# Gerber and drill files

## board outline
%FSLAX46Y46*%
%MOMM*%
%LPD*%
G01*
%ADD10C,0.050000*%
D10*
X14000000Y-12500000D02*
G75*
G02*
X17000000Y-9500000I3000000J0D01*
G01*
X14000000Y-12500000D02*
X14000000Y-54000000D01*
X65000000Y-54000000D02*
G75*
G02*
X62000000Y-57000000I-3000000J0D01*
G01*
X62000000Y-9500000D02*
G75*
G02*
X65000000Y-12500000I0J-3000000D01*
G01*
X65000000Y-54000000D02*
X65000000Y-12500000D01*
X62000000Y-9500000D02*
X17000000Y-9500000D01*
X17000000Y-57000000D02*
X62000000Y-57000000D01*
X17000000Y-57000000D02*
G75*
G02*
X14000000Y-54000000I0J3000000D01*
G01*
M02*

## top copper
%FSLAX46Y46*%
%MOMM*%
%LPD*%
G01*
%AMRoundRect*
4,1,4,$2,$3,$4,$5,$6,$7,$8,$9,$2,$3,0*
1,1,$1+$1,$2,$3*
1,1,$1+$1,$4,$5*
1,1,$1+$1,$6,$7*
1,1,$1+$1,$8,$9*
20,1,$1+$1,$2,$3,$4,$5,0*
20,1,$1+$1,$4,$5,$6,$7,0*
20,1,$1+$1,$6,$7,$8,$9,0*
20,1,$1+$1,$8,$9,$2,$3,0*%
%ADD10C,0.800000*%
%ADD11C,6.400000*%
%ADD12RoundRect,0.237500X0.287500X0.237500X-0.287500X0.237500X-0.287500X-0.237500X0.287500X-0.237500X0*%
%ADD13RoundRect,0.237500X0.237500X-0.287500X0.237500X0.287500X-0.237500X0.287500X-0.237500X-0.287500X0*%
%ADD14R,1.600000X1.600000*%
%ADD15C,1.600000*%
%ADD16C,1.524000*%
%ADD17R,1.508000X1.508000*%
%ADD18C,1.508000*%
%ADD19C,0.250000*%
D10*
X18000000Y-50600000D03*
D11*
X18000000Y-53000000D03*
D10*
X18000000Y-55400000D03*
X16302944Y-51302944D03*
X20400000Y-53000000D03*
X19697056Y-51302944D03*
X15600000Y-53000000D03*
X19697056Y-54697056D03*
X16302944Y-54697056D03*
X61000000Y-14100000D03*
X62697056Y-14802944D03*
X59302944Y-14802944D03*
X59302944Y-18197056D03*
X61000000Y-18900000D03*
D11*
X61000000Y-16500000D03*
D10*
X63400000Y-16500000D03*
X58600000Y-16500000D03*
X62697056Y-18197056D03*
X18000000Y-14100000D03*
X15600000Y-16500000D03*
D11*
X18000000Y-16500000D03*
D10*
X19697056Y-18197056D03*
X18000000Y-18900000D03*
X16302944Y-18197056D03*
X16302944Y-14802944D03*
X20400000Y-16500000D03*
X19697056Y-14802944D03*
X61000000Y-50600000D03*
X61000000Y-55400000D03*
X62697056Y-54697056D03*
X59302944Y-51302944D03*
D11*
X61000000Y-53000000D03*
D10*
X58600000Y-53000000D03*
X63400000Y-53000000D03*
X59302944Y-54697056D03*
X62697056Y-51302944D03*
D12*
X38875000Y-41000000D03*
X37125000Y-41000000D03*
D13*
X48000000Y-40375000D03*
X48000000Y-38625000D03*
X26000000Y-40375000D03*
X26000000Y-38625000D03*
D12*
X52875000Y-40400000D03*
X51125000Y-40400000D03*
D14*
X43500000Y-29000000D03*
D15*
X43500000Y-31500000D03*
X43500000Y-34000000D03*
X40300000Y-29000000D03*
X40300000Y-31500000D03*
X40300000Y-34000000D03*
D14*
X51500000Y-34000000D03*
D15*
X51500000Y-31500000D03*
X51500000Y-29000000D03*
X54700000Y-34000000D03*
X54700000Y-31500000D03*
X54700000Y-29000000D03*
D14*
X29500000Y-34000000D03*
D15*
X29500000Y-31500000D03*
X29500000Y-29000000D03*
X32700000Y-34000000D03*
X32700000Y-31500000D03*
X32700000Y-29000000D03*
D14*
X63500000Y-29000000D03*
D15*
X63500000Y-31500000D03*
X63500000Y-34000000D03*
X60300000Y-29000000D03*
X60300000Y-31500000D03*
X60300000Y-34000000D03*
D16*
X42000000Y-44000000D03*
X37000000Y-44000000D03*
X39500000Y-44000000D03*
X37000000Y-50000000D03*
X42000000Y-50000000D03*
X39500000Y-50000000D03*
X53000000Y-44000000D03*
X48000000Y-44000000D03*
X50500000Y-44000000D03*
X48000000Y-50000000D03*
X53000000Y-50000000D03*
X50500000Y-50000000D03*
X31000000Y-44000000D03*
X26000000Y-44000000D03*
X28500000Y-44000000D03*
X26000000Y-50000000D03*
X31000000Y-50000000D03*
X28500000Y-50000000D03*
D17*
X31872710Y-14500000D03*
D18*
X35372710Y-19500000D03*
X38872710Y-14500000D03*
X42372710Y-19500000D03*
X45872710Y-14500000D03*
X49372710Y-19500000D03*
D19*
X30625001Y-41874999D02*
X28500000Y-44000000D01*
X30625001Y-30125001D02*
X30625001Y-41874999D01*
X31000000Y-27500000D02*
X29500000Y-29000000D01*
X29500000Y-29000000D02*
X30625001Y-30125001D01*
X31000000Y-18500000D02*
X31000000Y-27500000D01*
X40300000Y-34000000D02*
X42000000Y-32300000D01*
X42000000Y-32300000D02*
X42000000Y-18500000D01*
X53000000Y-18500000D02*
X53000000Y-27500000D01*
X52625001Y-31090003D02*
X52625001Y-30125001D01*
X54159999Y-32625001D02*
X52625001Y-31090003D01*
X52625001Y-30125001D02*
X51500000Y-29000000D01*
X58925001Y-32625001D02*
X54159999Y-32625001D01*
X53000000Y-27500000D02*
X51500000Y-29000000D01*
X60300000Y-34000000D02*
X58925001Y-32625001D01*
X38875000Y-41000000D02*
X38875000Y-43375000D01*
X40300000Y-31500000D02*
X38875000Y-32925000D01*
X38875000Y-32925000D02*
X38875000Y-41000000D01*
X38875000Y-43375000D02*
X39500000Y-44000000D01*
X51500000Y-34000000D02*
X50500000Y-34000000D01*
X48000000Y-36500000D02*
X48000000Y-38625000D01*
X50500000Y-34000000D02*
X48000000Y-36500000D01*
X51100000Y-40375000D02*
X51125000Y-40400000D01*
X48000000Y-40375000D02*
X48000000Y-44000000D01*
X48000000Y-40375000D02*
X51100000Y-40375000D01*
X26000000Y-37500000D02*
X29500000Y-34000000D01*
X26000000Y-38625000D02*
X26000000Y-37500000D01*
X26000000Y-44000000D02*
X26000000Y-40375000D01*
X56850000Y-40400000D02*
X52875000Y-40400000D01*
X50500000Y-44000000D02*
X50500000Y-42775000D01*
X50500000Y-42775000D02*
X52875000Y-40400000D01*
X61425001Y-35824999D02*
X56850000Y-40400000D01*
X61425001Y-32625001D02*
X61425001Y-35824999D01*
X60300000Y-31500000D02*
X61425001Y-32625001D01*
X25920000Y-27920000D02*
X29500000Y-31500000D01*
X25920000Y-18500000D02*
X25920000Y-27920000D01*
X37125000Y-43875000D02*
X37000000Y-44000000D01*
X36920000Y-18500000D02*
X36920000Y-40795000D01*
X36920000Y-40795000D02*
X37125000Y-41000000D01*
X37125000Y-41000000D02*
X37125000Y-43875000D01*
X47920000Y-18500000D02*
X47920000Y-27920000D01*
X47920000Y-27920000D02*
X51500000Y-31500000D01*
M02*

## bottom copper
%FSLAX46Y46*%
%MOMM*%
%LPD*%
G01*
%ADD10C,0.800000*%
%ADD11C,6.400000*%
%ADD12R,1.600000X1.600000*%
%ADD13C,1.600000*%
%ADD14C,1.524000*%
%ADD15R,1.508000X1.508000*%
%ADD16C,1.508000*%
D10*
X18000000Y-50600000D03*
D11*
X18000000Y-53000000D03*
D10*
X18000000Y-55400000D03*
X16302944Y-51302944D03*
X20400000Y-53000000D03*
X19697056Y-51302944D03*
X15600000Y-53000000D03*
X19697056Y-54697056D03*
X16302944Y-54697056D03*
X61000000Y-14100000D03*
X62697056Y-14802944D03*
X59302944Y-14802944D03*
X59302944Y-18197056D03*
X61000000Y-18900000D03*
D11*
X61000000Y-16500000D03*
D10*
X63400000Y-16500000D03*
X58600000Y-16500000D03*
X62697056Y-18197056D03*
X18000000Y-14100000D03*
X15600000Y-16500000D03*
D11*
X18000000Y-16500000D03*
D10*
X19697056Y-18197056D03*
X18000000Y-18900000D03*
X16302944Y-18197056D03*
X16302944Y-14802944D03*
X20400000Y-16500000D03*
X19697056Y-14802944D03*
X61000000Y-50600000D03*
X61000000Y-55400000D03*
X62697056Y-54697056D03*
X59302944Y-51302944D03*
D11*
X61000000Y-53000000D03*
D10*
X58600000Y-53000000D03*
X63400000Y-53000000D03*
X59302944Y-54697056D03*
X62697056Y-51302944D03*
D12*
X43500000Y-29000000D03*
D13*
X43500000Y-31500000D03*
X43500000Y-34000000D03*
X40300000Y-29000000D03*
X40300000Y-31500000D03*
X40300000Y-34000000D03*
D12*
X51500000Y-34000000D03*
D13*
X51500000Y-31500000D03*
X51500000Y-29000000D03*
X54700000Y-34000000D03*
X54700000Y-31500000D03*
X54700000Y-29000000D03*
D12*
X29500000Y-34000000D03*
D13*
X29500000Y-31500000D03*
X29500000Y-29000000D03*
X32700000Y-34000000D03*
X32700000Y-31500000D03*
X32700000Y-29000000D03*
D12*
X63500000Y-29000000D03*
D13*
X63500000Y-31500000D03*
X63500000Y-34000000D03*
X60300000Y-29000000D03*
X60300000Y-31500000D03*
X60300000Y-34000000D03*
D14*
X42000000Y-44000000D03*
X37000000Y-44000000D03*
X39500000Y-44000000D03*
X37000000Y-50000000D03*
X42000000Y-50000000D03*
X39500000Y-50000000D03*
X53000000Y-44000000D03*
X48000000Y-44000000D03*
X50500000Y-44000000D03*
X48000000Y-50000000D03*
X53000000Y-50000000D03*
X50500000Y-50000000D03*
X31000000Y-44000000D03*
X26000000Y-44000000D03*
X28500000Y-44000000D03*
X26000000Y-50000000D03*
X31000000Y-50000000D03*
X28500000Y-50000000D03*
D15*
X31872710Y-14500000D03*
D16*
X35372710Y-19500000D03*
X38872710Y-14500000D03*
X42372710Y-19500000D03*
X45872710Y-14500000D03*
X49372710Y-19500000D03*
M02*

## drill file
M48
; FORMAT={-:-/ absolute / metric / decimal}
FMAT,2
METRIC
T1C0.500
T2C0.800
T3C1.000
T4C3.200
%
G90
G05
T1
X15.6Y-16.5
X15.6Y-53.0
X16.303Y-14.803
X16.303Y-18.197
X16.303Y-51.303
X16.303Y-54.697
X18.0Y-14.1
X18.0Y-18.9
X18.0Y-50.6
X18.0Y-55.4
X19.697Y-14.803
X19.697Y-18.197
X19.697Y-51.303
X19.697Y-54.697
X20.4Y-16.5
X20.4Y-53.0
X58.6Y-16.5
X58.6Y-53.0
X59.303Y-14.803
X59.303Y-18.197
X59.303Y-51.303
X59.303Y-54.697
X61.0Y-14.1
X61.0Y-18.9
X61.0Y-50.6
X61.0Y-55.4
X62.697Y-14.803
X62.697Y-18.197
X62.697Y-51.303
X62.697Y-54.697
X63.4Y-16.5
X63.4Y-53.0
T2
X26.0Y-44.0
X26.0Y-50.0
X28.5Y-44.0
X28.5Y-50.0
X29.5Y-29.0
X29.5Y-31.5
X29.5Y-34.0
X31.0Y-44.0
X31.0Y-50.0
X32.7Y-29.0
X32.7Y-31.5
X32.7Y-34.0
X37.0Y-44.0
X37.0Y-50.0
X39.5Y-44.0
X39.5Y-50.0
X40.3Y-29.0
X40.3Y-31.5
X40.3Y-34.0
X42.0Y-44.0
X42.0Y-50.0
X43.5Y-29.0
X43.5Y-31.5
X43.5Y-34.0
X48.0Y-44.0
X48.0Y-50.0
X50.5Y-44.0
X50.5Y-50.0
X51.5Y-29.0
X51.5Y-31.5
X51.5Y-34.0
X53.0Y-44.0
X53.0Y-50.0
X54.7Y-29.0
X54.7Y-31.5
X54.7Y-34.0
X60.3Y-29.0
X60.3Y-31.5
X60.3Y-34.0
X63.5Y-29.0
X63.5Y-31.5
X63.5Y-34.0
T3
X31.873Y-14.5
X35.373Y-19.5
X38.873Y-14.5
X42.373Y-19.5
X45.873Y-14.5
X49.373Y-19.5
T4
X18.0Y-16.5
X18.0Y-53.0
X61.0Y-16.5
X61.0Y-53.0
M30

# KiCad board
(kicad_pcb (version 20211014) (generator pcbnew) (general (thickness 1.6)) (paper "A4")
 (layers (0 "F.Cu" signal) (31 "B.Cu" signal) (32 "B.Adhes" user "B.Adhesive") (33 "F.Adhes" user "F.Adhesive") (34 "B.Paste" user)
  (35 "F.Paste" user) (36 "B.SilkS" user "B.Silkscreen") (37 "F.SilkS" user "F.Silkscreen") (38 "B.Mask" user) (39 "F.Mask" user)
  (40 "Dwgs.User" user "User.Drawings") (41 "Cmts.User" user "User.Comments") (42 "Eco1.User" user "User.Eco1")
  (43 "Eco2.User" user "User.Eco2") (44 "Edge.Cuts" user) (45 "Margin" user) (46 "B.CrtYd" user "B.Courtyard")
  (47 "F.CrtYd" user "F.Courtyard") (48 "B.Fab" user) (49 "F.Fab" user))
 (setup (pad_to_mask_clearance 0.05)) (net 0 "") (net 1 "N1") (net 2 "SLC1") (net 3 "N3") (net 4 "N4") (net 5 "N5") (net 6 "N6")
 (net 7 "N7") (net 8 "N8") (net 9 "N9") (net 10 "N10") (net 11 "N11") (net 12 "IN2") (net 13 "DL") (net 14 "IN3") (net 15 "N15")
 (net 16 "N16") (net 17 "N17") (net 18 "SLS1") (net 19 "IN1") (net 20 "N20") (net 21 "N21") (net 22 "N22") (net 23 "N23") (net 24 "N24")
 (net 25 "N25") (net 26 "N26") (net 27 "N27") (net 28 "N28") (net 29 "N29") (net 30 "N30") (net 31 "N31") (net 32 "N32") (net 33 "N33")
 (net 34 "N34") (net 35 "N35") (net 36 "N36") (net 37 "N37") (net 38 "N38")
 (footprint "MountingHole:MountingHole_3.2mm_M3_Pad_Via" (layer "F.Cu") (at 18 53)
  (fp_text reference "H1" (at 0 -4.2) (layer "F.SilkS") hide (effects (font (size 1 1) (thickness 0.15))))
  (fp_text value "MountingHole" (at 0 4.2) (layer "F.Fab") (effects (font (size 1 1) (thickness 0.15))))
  (pad "1" thru_hole circle locked (at 0 -2.4) (size 0.8 0.8) (drill 0.5) (layers *.Cu *.Mask))
  (pad "1" thru_hole circle locked (at 0 0) (size 6.4 6.4) (drill 3.2) (layers *.Cu *.Mask))
  (pad "1" thru_hole circle locked (at 0 2.4) (size 0.8 0.8) (drill 0.5) (layers *.Cu *.Mask))
  (pad "1" thru_hole circle locked (at -1.697056 -1.697056) (size 0.8 0.8) (drill 0.5) (layers *.Cu *.Mask))
  (pad "1" thru_hole circle locked (at 2.4 0) (size 0.8 0.8) (drill 0.5) (layers *.Cu *.Mask))
  (pad "1" thru_hole circle locked (at 1.697056 -1.697056) (size 0.8 0.8) (drill 0.5) (layers *.Cu *.Mask))
  (pad "1" thru_hole circle locked (at -2.4 0) (size 0.8 0.8) (drill 0.5) (layers *.Cu *.Mask))
  (pad "1" thru_hole circle locked (at 1.697056 1.697056) (size 0.8 0.8) (drill 0.5) (layers *.Cu *.Mask))
  (pad "1" thru_hole circle locked (at -1.697056 1.697056) (size 0.8 0.8) (drill 0.5) (layers *.Cu *.Mask)))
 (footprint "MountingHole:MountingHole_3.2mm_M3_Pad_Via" (layer "F.Cu") (at 61 16.5)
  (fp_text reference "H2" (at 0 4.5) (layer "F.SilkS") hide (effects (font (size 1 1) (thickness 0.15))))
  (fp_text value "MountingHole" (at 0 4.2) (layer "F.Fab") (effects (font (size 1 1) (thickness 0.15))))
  (pad "1" thru_hole circle locked (at 0 -2.4) (size 0.8 0.8) (drill 0.5) (layers *.Cu *.Mask))
  (pad "1" thru_hole circle locked (at 1.697056 -1.697056) (size 0.8 0.8) (drill 0.5) (layers *.Cu *.Mask))
  (pad "1" thru_hole circle locked (at -1.697056 -1.697056) (size 0.8 0.8) (drill 0.5) (layers *.Cu *.Mask))
  (pad "1" thru_hole circle locked (at -1.697056 1.697056) (size 0.8 0.8) (drill 0.5) (layers *.Cu *.Mask))
  (pad "1" thru_hole circle locked (at 0 2.4) (size 0.8 0.8) (drill 0.5) (layers *.Cu *.Mask))
  (pad "1" thru_hole circle locked (at 0 0) (size 6.4 6.4) (drill 3.2) (layers *.Cu *.Mask))
  (pad "1" thru_hole circle locked (at 2.4 0) (size 0.8 0.8) (drill 0.5) (layers *.Cu *.Mask))
  (pad "1" thru_hole circle locked (at -2.4 0) (size 0.8 0.8) (drill 0.5) (layers *.Cu *.Mask))
  (pad "1" thru_hole circle locked (at 1.697056 1.697056) (size 0.8 0.8) (drill 0.5) (layers *.Cu *.Mask)))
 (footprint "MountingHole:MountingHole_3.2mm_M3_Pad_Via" (layer "F.Cu") (at 18 16.5)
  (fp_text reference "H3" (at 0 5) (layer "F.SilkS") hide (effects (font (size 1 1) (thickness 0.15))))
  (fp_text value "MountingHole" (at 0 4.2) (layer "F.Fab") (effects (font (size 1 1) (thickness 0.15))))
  (pad "1" thru_hole circle locked (at 0 -2.4) (size 0.8 0.8) (drill 0.5) (layers *.Cu *.Mask))
  (pad "1" thru_hole circle locked (at -2.4 0) (size 0.8 0.8) (drill 0.5) (layers *.Cu *.Mask))
  (pad "1" thru_hole circle locked (at 0 0) (size 6.4 6.4) (drill 3.2) (layers *.Cu *.Mask))
  (pad "1" thru_hole circle locked (at 1.697056 1.697056) (size 0.8 0.8) (drill 0.5) (layers *.Cu *.Mask))
  (pad "1" thru_hole circle locked (at 0 2.4) (size 0.8 0.8) (drill 0.5) (layers *.Cu *.Mask))
  (pad "1" thru_hole circle locked (at -1.697056 1.697056) (size 0.8 0.8) (drill 0.5) (layers *.Cu *.Mask))
  (pad "1" thru_hole circle locked (at -1.697056 -1.697056) (size 0.8 0.8) (drill 0.5) (layers *.Cu *.Mask))
  (pad "1" thru_hole circle locked (at 2.4 0) (size 0.8 0.8) (drill 0.5) (layers *.Cu *.Mask))
  (pad "1" thru_hole circle locked (at 1.697056 -1.697056) (size 0.8 0.8) (drill 0.5) (layers *.Cu *.Mask)))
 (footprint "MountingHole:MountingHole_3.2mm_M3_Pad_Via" (layer "F.Cu") (at 61 53)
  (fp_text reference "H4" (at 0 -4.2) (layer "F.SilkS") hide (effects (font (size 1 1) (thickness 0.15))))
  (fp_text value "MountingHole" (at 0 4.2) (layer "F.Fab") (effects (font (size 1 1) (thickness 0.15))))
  (pad "1" thru_hole circle locked (at 0 -2.4) (size 0.8 0.8) (drill 0.5) (layers *.Cu *.Mask))
  (pad "1" thru_hole circle locked (at 0 2.4) (size 0.8 0.8) (drill 0.5) (layers *.Cu *.Mask))
  (pad "1" thru_hole circle locked (at 1.697056 1.697056) (size 0.8 0.8) (drill 0.5) (layers *.Cu *.Mask))
  (pad "1" thru_hole circle locked (at -1.697056 -1.697056) (size 0.8 0.8) (drill 0.5) (layers *.Cu *.Mask))
  (pad "1" thru_hole circle locked (at 0 0) (size 6.4 6.4) (drill 3.2) (layers *.Cu *.Mask))
  (pad "1" thru_hole circle locked (at -2.4 0) (size 0.8 0.8) (drill 0.5) (layers *.Cu *.Mask))
  (pad "1" thru_hole circle locked (at 2.4 0) (size 0.8 0.8) (drill 0.5) (layers *.Cu *.Mask))
  (pad "1" thru_hole circle locked (at -1.697056 1.697056) (size 0.8 0.8) (drill 0.5) (layers *.Cu *.Mask))
  (pad "1" thru_hole circle locked (at 1.697056 -1.697056) (size 0.8 0.8) (drill 0.5) (layers *.Cu *.Mask)))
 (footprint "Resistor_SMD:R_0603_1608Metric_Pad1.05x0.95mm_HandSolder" (layer "F.Cu") (at 38 41 180)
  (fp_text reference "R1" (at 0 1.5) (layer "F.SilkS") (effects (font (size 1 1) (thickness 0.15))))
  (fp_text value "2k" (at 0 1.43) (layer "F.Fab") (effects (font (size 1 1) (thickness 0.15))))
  (pad "1" smd roundrect locked (at -0.875 0 180) (size 1.05 0.95) (layers "F.Cu" "F.Paste" "F.Mask") (roundrect_rratio 0.25) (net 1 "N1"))
  (pad "2" smd roundrect locked (at 0.875 0 180) (size 1.05 0.95) (layers "F.Cu" "F.Paste" "F.Mask") (roundrect_rratio 0.25) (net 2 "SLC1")))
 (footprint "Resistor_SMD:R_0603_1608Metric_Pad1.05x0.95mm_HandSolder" (layer "F.Cu") (at 48 39.5 90)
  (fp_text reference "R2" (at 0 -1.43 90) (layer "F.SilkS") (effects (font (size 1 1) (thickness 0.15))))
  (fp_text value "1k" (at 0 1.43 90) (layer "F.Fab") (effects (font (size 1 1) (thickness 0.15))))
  (pad "1" smd roundrect locked (at -0.875 0 90) (size 1.05 0.95) (layers "F.Cu" "F.Paste" "F.Mask") (roundrect_rratio 0.25) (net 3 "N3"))
  (pad "2" smd roundrect locked (at 0.875 0 90) (size 1.05 0.95) (layers "F.Cu" "F.Paste" "F.Mask") (roundrect_rratio 0.25) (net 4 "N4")))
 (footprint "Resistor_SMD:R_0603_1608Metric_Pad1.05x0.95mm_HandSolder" (layer "F.Cu") (at 26 39.5 90)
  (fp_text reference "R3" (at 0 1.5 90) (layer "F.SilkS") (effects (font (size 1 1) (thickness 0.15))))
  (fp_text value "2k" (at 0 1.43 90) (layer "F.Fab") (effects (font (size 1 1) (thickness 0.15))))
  (pad "1" smd roundrect locked (at -0.875 0 90) (size 1.05 0.95) (layers "F.Cu" "F.Paste" "F.Mask") (roundrect_rratio 0.25) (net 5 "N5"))
  (pad "2" smd roundrect locked (at 0.875 0 90) (size 1.05 0.95) (layers "F.Cu" "F.Paste" "F.Mask") (roundrect_rratio 0.25) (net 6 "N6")))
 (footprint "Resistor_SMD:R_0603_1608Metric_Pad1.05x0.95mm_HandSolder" (layer "F.Cu") (at 52 40.4 180)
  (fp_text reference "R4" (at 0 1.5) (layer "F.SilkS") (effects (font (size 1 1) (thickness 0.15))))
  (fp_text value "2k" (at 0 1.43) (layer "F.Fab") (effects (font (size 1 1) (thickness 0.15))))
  (pad "1" smd roundrect locked (at -0.875 0 180) (size 1.05 0.95) (layers "F.Cu" "F.Paste" "F.Mask") (roundrect_rratio 0.25) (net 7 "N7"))
  (pad "2" smd roundrect locked (at 0.875 0 180) (size 1.05 0.95) (layers "F.Cu" "F.Paste" "F.Mask") (roundrect_rratio 0.25) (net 3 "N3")))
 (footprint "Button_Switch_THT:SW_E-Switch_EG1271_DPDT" (layer "F.Cu") (at 43.5 29 -90)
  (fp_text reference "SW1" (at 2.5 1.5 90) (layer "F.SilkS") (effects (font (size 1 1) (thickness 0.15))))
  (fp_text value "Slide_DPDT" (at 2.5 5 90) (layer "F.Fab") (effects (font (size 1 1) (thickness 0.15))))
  (pad "1" thru_hole rect locked (at 0 0 270) (size 1.6 1.6) (drill 0.8) (layers *.Cu *.Mask) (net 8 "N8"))
  (pad "2" thru_hole circle locked (at 2.5 0 270) (size 1.6 1.6) (drill 0.8) (layers *.Cu *.Mask) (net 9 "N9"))
  (pad "3" thru_hole circle locked (at 5 0 270) (size 1.6 1.6) (drill 0.8) (layers *.Cu *.Mask) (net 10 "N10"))
  (pad "4" thru_hole circle locked (at 0 3.2 270) (size 1.6 1.6) (drill 0.8) (layers *.Cu *.Mask) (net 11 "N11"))
  (pad "5" thru_hole circle locked (at 2.5 3.2 270) (size 1.6 1.6) (drill 0.8) (layers *.Cu *.Mask) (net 1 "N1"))
  (pad "6" thru_hole circle locked (at 5 3.2 270) (size 1.6 1.6) (drill 0.8) (layers *.Cu *.Mask) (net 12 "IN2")))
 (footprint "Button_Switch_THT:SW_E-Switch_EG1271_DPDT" (layer "F.Cu") (at 51.5 34 90)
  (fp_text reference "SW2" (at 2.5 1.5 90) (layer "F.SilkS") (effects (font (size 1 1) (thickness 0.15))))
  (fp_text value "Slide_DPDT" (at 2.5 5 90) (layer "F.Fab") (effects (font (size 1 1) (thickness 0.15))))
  (pad "1" thru_hole rect locked (at 0 0 90) (size 1.6 1.6) (drill 0.8) (layers *.Cu *.Mask) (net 4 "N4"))
  (pad "2" thru_hole circle locked (at 2.5 0 90) (size 1.6 1.6) (drill 0.8) (layers *.Cu *.Mask) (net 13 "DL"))
  (pad "3" thru_hole circle locked (at 5 0 90) (size 1.6 1.6) (drill 0.8) (layers *.Cu *.Mask) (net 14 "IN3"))
  (pad "4" thru_hole circle locked (at 0 3.2 90) (size 1.6 1.6) (drill 0.8) (layers *.Cu *.Mask) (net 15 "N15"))
  (pad "5" thru_hole circle locked (at 2.5 3.2 90) (size 1.6 1.6) (drill 0.8) (layers *.Cu *.Mask) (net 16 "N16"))
  (pad "6" thru_hole circle locked (at 5 3.2 90) (size 1.6 1.6) (drill 0.8) (layers *.Cu *.Mask) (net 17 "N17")))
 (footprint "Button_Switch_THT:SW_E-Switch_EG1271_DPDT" (layer "F.Cu") (at 29.5 34 90)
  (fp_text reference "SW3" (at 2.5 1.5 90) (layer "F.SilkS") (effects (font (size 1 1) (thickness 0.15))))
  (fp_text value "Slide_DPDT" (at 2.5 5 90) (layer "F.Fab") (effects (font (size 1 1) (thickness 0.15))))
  (pad "1" thru_hole rect locked (at 0 0 90) (size 1.6 1.6) (drill 0.8) (layers *.Cu *.Mask) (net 6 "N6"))
  (pad "2" thru_hole circle locked (at 2.5 0 90) (size 1.6 1.6) (drill 0.8) (layers *.Cu *.Mask) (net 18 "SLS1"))
  (pad "3" thru_hole circle locked (at 5 0 90) (size 1.6 1.6) (drill 0.8) (layers *.Cu *.Mask) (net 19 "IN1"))
  (pad "4" thru_hole circle locked (at 0 3.2 90) (size 1.6 1.6) (drill 0.8) (layers *.Cu *.Mask) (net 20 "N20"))
  (pad "5" thru_hole circle locked (at 2.5 3.2 90) (size 1.6 1.6) (drill 0.8) (layers *.Cu *.Mask) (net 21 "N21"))
  (pad "6" thru_hole circle locked (at 5 3.2 90) (size 1.6 1.6) (drill 0.8) (layers *.Cu *.Mask) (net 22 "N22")))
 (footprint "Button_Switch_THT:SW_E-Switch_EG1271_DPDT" (layer "F.Cu") (at 63.5 29 -90)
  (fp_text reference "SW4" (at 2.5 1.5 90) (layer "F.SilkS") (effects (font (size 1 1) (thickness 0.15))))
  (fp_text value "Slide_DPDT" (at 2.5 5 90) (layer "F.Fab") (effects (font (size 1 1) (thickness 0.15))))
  (pad "1" thru_hole rect locked (at 0 0 270) (size 1.6 1.6) (drill 0.8) (layers *.Cu *.Mask) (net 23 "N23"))
  (pad "2" thru_hole circle locked (at 2.5 0 270) (size 1.6 1.6) (drill 0.8) (layers *.Cu *.Mask) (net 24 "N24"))
  (pad "3" thru_hole circle locked (at 5 0 270) (size 1.6 1.6) (drill 0.8) (layers *.Cu *.Mask) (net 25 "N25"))
  (pad "4" thru_hole circle locked (at 0 3.2 270) (size 1.6 1.6) (drill 0.8) (layers *.Cu *.Mask) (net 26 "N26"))
  (pad "5" thru_hole circle locked (at 2.5 3.2 270) (size 1.6 1.6) (drill 0.8) (layers *.Cu *.Mask) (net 7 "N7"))
  (pad "6" thru_hole circle locked (at 5 3.2 270) (size 1.6 1.6) (drill 0.8) (layers *.Cu *.Mask) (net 14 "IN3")))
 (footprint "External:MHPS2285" (layer "F.Cu") (at 40.5 48)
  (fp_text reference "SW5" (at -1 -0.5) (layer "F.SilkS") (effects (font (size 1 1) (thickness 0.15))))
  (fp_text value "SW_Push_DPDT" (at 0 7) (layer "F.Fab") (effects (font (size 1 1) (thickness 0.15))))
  (pad "1" thru_hole circle locked (at 1.5 -4) (size 1.524 1.524) (drill 0.8) (layers *.Cu *.Mask) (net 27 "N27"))
  (pad "2" thru_hole circle locked (at -3.5 -4) (size 1.524 1.524) (drill 0.8) (layers *.Cu *.Mask) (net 2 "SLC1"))
  (pad "3" thru_hole circle locked (at -1 -4) (size 1.524 1.524) (drill 0.8) (layers *.Cu *.Mask) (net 1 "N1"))
  (pad "4" thru_hole circle locked (at -3.5 2) (size 1.524 1.524) (drill 0.8) (layers *.Cu *.Mask) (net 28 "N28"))
  (pad "5" thru_hole circle locked (at 1.5 2) (size 1.524 1.524) (drill 0.8) (layers *.Cu *.Mask) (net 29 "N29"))
  (pad "6" thru_hole circle locked (at -1 2) (size 1.524 1.524) (drill 0.8) (layers *.Cu *.Mask) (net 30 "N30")))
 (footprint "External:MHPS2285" (layer "F.Cu") (at 51.5 48)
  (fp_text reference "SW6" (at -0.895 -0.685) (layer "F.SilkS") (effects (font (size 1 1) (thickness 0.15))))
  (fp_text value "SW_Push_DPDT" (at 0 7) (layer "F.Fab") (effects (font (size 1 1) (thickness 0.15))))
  (pad "1" thru_hole circle locked (at 1.5 -4) (size 1.524 1.524) (drill 0.8) (layers *.Cu *.Mask) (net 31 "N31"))
  (pad "2" thru_hole circle locked (at -3.5 -4) (size 1.524 1.524) (drill 0.8) (layers *.Cu *.Mask) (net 3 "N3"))
  (pad "3" thru_hole circle locked (at -1 -4) (size 1.524 1.524) (drill 0.8) (layers *.Cu *.Mask) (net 7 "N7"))
  (pad "4" thru_hole circle locked (at -3.5 2) (size 1.524 1.524) (drill 0.8) (layers *.Cu *.Mask) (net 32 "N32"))
  (pad "5" thru_hole circle locked (at 1.5 2) (size 1.524 1.524) (drill 0.8) (layers *.Cu *.Mask) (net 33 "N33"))
  (pad "6" thru_hole circle locked (at -1 2) (size 1.524 1.524) (drill 0.8) (layers *.Cu *.Mask) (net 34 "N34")))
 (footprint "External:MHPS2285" (layer "F.Cu") (at 29.5 48)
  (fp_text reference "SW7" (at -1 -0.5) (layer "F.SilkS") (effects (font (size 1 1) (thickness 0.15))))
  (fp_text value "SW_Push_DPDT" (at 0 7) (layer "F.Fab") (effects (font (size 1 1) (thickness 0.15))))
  (pad "1" thru_hole circle locked (at 1.5 -4) (size 1.524 1.524) (drill 0.8) (layers *.Cu *.Mask) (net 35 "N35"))
  (pad "2" thru_hole circle locked (at -3.5 -4) (size 1.524 1.524) (drill 0.8) (layers *.Cu *.Mask) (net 5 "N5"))
  (pad "3" thru_hole circle locked (at -1 -4) (size 1.524 1.524) (drill 0.8) (layers *.Cu *.Mask) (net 19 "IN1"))
  (pad "4" thru_hole circle locked (at -3.5 2) (size 1.524 1.524) (drill 0.8) (layers *.Cu *.Mask) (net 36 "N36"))
  (pad "5" thru_hole circle locked (at 1.5 2) (size 1.524 1.524) (drill 0.8) (layers *.Cu *.Mask) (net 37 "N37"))
  (pad "6" thru_hole circle locked (at -1 2) (size 1.524 1.524) (drill 0.8) (layers *.Cu *.Mask) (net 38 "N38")))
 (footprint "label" (layer "F.Cu") (at 26 29)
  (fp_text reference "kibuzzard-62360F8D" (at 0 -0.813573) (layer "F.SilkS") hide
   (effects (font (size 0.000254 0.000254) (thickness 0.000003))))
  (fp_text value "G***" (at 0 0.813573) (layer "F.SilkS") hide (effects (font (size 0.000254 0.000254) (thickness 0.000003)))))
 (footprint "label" (layer "F.Cu") (at 48 29)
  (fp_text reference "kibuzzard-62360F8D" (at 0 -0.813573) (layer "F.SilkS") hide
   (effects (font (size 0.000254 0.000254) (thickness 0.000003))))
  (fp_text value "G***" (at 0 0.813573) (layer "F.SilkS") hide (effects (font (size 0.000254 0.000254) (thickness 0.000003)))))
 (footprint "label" (layer "F.Cu") (at 37.5 29)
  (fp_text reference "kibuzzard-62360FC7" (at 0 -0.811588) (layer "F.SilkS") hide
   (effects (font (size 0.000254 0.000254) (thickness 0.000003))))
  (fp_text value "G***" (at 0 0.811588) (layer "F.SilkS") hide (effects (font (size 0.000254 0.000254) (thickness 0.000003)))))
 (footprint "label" (layer "F.Cu") (at 57.5 29)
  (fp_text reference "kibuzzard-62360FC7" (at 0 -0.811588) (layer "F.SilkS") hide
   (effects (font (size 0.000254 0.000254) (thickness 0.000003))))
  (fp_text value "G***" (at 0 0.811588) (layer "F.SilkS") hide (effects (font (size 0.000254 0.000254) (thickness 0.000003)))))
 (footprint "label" (layer "F.Cu") (at 26.05 52.5)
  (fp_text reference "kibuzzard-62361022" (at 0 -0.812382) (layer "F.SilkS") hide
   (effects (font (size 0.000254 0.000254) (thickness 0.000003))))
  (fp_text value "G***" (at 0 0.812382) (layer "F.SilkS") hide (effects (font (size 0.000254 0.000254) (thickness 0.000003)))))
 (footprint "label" (layer "F.Cu") (at 37.05 52.5)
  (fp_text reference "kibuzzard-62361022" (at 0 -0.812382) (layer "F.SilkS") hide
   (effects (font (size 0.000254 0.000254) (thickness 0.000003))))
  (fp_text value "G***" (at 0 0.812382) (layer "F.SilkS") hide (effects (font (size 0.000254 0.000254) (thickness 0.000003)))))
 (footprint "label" (layer "F.Cu") (at 48.05 52.5)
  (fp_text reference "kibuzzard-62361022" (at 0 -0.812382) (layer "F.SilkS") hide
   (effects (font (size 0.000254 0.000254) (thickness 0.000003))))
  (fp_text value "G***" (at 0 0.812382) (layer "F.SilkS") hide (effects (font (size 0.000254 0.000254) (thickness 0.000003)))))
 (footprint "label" (layer "F.Cu") (at 41.75 52.5)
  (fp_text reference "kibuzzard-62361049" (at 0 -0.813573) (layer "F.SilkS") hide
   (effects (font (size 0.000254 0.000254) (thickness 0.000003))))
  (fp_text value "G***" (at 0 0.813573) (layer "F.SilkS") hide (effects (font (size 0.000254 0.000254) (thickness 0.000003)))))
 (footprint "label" (layer "F.Cu") (at 52.75 52.5)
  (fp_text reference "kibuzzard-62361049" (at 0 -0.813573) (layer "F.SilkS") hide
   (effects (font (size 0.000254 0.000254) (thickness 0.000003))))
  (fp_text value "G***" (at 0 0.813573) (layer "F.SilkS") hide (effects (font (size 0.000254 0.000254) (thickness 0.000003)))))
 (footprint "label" (layer "F.Cu") (at 30.75 52.5)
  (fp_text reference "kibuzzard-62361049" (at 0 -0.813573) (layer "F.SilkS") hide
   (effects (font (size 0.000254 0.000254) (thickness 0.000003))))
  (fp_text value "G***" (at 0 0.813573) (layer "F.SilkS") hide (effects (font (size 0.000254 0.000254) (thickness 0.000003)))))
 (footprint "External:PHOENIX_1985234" (layer "F.Cu") (at 31.87271 14.5)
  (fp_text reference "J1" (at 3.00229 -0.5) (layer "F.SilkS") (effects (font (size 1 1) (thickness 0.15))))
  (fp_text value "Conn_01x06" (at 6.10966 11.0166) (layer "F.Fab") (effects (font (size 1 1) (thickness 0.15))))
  (pad "1" thru_hole rect locked (at 0 0) (size 1.508 1.508) (drill 1) (layers *.Cu *.Mask) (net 18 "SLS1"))
  (pad "2" thru_hole circle locked (at 3.5 5) (size 1.508 1.508) (drill 1) (layers *.Cu *.Mask) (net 19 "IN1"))
  (pad "3" thru_hole circle locked (at 7 0) (size 1.508 1.508) (drill 1) (layers *.Cu *.Mask) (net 2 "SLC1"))
  (pad "4" thru_hole circle locked (at 10.5 5) (size 1.508 1.508) (drill 1) (layers *.Cu *.Mask) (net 12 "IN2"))
  (pad "5" thru_hole circle locked (at 14 0) (size 1.508 1.508) (drill 1) (layers *.Cu *.Mask) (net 13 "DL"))
  (pad "6" thru_hole circle locked (at 17.5 5) (size 1.508 1.508) (drill 1) (layers *.Cu *.Mask) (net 14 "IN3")))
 (gr_arc (start 14 12.5) (mid 14.87868 10.37868) (end 17 9.5) (layer "Edge.Cuts") (width 0.05))
 (gr_line (start 14 12.5) (end 14 54) (layer "Edge.Cuts") (width 0.05))
 (gr_arc (start 65 54) (mid 64.12132 56.12132) (end 62 57) (layer "Edge.Cuts") (width 0.05))
 (gr_arc (start 62 9.5) (mid 64.12132 10.37868) (end 65 12.5) (layer "Edge.Cuts") (width 0.05))
 (gr_line (start 65 54) (end 65 12.5) (layer "Edge.Cuts") (width 0.05))
 (gr_line (start 62 9.5) (end 17 9.5) (layer "Edge.Cuts") (width 0.05))
 (gr_line (start 17 57) (end 62 57) (layer "Edge.Cuts") (width 0.05))
 (gr_arc (start 17 57) (mid 14.87868 56.12132) (end 14 54) (layer "Edge.Cuts") (width 0.05))
 (segment (start 30.625001 41.874999) (end 28.5 44) (width 0.25) (layer "F.Cu") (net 19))
 (segment (start 30.625001 30.125001) (end 30.625001 41.874999) (width 0.25) (layer "F.Cu") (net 19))
 (segment (start 31 27.5) (end 29.5 29) (width 0.25) (layer "F.Cu") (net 19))
 (segment (start 29.5 29) (end 30.625001 30.125001) (width 0.25) (layer "F.Cu") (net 19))
 (segment (start 31 18.5) (end 31 27.5) (width 0.25) (layer "F.Cu") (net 19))
 (segment (start 40.3 34) (end 42 32.3) (width 0.25) (layer "F.Cu") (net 12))
 (segment (start 42 32.3) (end 42 18.5) (width 0.25) (layer "F.Cu") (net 12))
 (segment (start 53 18.5) (end 53 27.5) (width 0.25) (layer "F.Cu") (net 14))
 (segment (start 52.625001 31.090003) (end 52.625001 30.125001) (width 0.25) (layer "F.Cu") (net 14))
 (segment (start 54.159999 32.625001) (end 52.625001 31.090003) (width 0.25) (layer "F.Cu") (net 14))
 (segment (start 52.625001 30.125001) (end 51.5 29) (width 0.25) (layer "F.Cu") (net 14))
 (segment (start 58.925001 32.625001) (end 54.159999 32.625001) (width 0.25) (layer "F.Cu") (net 14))
 (segment (start 53 27.5) (end 51.5 29) (width 0.25) (layer "F.Cu") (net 14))
 (segment (start 60.3 34) (end 58.925001 32.625001) (width 0.25) (layer "F.Cu") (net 14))
 (segment (start 38.875 41) (end 38.875 43.375) (width 0.25) (layer "F.Cu") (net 1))
 (segment (start 40.3 31.5) (end 38.875 32.925) (width 0.25) (layer "F.Cu") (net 1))
 (segment (start 38.875 32.925) (end 38.875 41) (width 0.25) (layer "F.Cu") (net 1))
 (segment (start 38.875 43.375) (end 39.5 44) (width 0.25) (layer "F.Cu") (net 1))
 (segment (start 51.5 34) (end 50.5 34) (width 0.25) (layer "F.Cu") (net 4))
 (segment (start 48 36.5) (end 48 38.625) (width 0.25) (layer "F.Cu") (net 4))
 (segment (start 50.5 34) (end 48 36.5) (width 0.25) (layer "F.Cu") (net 4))
 (segment (start 51.1 40.375) (end 51.125 40.4) (width 0.25) (layer "F.Cu") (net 3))
 (segment (start 48 40.375) (end 48 44) (width 0.25) (layer "F.Cu") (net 3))
 (segment (start 48 40.375) (end 51.1 40.375) (width 0.25) (layer "F.Cu") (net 3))
 (segment (start 26 37.5) (end 29.5 34) (width 0.25) (layer "F.Cu") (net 6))
 (segment (start 26 38.625) (end 26 37.5) (width 0.25) (layer "F.Cu") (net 6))
 (segment (start 26 44) (end 26 40.375) (width 0.25) (layer "F.Cu") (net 5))
 (segment (start 56.85 40.4) (end 52.875 40.4) (width 0.25) (layer "F.Cu") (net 7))
 (segment (start 50.5 44) (end 50.5 42.775) (width 0.25) (layer "F.Cu") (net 7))
 (segment (start 50.5 42.775) (end 52.875 40.4) (width 0.25) (layer "F.Cu") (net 7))
 (segment (start 61.425001 35.824999) (end 56.85 40.4) (width 0.25) (layer "F.Cu") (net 7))
 (segment (start 61.425001 32.625001) (end 61.425001 35.824999) (width 0.25) (layer "F.Cu") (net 7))
 (segment (start 60.3 31.5) (end 61.425001 32.625001) (width 0.25) (layer "F.Cu") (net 7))
 (segment (start 25.92 27.92) (end 29.5 31.5) (width 0.25) (layer "F.Cu") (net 18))
 (segment (start 25.92 18.5) (end 25.92 27.92) (width 0.25) (layer "F.Cu") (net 18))
 (segment (start 37.125 43.875) (end 37 44) (width 0.25) (layer "F.Cu") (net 2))
 (segment (start 36.92 18.5) (end 36.92 40.795) (width 0.25) (layer "F.Cu") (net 2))
 (segment (start 36.92 40.795) (end 37.125 41) (width 0.25) (layer "F.Cu") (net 2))
 (segment (start 37.125 41) (end 37.125 43.875) (width 0.25) (layer "F.Cu") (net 2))
 (segment (start 47.92 18.5) (end 47.92 27.92) (width 0.25) (layer "F.Cu") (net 13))
 (segment (start 47.92 27.92) (end 51.5 31.5) (width 0.25) (layer "F.Cu") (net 13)))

